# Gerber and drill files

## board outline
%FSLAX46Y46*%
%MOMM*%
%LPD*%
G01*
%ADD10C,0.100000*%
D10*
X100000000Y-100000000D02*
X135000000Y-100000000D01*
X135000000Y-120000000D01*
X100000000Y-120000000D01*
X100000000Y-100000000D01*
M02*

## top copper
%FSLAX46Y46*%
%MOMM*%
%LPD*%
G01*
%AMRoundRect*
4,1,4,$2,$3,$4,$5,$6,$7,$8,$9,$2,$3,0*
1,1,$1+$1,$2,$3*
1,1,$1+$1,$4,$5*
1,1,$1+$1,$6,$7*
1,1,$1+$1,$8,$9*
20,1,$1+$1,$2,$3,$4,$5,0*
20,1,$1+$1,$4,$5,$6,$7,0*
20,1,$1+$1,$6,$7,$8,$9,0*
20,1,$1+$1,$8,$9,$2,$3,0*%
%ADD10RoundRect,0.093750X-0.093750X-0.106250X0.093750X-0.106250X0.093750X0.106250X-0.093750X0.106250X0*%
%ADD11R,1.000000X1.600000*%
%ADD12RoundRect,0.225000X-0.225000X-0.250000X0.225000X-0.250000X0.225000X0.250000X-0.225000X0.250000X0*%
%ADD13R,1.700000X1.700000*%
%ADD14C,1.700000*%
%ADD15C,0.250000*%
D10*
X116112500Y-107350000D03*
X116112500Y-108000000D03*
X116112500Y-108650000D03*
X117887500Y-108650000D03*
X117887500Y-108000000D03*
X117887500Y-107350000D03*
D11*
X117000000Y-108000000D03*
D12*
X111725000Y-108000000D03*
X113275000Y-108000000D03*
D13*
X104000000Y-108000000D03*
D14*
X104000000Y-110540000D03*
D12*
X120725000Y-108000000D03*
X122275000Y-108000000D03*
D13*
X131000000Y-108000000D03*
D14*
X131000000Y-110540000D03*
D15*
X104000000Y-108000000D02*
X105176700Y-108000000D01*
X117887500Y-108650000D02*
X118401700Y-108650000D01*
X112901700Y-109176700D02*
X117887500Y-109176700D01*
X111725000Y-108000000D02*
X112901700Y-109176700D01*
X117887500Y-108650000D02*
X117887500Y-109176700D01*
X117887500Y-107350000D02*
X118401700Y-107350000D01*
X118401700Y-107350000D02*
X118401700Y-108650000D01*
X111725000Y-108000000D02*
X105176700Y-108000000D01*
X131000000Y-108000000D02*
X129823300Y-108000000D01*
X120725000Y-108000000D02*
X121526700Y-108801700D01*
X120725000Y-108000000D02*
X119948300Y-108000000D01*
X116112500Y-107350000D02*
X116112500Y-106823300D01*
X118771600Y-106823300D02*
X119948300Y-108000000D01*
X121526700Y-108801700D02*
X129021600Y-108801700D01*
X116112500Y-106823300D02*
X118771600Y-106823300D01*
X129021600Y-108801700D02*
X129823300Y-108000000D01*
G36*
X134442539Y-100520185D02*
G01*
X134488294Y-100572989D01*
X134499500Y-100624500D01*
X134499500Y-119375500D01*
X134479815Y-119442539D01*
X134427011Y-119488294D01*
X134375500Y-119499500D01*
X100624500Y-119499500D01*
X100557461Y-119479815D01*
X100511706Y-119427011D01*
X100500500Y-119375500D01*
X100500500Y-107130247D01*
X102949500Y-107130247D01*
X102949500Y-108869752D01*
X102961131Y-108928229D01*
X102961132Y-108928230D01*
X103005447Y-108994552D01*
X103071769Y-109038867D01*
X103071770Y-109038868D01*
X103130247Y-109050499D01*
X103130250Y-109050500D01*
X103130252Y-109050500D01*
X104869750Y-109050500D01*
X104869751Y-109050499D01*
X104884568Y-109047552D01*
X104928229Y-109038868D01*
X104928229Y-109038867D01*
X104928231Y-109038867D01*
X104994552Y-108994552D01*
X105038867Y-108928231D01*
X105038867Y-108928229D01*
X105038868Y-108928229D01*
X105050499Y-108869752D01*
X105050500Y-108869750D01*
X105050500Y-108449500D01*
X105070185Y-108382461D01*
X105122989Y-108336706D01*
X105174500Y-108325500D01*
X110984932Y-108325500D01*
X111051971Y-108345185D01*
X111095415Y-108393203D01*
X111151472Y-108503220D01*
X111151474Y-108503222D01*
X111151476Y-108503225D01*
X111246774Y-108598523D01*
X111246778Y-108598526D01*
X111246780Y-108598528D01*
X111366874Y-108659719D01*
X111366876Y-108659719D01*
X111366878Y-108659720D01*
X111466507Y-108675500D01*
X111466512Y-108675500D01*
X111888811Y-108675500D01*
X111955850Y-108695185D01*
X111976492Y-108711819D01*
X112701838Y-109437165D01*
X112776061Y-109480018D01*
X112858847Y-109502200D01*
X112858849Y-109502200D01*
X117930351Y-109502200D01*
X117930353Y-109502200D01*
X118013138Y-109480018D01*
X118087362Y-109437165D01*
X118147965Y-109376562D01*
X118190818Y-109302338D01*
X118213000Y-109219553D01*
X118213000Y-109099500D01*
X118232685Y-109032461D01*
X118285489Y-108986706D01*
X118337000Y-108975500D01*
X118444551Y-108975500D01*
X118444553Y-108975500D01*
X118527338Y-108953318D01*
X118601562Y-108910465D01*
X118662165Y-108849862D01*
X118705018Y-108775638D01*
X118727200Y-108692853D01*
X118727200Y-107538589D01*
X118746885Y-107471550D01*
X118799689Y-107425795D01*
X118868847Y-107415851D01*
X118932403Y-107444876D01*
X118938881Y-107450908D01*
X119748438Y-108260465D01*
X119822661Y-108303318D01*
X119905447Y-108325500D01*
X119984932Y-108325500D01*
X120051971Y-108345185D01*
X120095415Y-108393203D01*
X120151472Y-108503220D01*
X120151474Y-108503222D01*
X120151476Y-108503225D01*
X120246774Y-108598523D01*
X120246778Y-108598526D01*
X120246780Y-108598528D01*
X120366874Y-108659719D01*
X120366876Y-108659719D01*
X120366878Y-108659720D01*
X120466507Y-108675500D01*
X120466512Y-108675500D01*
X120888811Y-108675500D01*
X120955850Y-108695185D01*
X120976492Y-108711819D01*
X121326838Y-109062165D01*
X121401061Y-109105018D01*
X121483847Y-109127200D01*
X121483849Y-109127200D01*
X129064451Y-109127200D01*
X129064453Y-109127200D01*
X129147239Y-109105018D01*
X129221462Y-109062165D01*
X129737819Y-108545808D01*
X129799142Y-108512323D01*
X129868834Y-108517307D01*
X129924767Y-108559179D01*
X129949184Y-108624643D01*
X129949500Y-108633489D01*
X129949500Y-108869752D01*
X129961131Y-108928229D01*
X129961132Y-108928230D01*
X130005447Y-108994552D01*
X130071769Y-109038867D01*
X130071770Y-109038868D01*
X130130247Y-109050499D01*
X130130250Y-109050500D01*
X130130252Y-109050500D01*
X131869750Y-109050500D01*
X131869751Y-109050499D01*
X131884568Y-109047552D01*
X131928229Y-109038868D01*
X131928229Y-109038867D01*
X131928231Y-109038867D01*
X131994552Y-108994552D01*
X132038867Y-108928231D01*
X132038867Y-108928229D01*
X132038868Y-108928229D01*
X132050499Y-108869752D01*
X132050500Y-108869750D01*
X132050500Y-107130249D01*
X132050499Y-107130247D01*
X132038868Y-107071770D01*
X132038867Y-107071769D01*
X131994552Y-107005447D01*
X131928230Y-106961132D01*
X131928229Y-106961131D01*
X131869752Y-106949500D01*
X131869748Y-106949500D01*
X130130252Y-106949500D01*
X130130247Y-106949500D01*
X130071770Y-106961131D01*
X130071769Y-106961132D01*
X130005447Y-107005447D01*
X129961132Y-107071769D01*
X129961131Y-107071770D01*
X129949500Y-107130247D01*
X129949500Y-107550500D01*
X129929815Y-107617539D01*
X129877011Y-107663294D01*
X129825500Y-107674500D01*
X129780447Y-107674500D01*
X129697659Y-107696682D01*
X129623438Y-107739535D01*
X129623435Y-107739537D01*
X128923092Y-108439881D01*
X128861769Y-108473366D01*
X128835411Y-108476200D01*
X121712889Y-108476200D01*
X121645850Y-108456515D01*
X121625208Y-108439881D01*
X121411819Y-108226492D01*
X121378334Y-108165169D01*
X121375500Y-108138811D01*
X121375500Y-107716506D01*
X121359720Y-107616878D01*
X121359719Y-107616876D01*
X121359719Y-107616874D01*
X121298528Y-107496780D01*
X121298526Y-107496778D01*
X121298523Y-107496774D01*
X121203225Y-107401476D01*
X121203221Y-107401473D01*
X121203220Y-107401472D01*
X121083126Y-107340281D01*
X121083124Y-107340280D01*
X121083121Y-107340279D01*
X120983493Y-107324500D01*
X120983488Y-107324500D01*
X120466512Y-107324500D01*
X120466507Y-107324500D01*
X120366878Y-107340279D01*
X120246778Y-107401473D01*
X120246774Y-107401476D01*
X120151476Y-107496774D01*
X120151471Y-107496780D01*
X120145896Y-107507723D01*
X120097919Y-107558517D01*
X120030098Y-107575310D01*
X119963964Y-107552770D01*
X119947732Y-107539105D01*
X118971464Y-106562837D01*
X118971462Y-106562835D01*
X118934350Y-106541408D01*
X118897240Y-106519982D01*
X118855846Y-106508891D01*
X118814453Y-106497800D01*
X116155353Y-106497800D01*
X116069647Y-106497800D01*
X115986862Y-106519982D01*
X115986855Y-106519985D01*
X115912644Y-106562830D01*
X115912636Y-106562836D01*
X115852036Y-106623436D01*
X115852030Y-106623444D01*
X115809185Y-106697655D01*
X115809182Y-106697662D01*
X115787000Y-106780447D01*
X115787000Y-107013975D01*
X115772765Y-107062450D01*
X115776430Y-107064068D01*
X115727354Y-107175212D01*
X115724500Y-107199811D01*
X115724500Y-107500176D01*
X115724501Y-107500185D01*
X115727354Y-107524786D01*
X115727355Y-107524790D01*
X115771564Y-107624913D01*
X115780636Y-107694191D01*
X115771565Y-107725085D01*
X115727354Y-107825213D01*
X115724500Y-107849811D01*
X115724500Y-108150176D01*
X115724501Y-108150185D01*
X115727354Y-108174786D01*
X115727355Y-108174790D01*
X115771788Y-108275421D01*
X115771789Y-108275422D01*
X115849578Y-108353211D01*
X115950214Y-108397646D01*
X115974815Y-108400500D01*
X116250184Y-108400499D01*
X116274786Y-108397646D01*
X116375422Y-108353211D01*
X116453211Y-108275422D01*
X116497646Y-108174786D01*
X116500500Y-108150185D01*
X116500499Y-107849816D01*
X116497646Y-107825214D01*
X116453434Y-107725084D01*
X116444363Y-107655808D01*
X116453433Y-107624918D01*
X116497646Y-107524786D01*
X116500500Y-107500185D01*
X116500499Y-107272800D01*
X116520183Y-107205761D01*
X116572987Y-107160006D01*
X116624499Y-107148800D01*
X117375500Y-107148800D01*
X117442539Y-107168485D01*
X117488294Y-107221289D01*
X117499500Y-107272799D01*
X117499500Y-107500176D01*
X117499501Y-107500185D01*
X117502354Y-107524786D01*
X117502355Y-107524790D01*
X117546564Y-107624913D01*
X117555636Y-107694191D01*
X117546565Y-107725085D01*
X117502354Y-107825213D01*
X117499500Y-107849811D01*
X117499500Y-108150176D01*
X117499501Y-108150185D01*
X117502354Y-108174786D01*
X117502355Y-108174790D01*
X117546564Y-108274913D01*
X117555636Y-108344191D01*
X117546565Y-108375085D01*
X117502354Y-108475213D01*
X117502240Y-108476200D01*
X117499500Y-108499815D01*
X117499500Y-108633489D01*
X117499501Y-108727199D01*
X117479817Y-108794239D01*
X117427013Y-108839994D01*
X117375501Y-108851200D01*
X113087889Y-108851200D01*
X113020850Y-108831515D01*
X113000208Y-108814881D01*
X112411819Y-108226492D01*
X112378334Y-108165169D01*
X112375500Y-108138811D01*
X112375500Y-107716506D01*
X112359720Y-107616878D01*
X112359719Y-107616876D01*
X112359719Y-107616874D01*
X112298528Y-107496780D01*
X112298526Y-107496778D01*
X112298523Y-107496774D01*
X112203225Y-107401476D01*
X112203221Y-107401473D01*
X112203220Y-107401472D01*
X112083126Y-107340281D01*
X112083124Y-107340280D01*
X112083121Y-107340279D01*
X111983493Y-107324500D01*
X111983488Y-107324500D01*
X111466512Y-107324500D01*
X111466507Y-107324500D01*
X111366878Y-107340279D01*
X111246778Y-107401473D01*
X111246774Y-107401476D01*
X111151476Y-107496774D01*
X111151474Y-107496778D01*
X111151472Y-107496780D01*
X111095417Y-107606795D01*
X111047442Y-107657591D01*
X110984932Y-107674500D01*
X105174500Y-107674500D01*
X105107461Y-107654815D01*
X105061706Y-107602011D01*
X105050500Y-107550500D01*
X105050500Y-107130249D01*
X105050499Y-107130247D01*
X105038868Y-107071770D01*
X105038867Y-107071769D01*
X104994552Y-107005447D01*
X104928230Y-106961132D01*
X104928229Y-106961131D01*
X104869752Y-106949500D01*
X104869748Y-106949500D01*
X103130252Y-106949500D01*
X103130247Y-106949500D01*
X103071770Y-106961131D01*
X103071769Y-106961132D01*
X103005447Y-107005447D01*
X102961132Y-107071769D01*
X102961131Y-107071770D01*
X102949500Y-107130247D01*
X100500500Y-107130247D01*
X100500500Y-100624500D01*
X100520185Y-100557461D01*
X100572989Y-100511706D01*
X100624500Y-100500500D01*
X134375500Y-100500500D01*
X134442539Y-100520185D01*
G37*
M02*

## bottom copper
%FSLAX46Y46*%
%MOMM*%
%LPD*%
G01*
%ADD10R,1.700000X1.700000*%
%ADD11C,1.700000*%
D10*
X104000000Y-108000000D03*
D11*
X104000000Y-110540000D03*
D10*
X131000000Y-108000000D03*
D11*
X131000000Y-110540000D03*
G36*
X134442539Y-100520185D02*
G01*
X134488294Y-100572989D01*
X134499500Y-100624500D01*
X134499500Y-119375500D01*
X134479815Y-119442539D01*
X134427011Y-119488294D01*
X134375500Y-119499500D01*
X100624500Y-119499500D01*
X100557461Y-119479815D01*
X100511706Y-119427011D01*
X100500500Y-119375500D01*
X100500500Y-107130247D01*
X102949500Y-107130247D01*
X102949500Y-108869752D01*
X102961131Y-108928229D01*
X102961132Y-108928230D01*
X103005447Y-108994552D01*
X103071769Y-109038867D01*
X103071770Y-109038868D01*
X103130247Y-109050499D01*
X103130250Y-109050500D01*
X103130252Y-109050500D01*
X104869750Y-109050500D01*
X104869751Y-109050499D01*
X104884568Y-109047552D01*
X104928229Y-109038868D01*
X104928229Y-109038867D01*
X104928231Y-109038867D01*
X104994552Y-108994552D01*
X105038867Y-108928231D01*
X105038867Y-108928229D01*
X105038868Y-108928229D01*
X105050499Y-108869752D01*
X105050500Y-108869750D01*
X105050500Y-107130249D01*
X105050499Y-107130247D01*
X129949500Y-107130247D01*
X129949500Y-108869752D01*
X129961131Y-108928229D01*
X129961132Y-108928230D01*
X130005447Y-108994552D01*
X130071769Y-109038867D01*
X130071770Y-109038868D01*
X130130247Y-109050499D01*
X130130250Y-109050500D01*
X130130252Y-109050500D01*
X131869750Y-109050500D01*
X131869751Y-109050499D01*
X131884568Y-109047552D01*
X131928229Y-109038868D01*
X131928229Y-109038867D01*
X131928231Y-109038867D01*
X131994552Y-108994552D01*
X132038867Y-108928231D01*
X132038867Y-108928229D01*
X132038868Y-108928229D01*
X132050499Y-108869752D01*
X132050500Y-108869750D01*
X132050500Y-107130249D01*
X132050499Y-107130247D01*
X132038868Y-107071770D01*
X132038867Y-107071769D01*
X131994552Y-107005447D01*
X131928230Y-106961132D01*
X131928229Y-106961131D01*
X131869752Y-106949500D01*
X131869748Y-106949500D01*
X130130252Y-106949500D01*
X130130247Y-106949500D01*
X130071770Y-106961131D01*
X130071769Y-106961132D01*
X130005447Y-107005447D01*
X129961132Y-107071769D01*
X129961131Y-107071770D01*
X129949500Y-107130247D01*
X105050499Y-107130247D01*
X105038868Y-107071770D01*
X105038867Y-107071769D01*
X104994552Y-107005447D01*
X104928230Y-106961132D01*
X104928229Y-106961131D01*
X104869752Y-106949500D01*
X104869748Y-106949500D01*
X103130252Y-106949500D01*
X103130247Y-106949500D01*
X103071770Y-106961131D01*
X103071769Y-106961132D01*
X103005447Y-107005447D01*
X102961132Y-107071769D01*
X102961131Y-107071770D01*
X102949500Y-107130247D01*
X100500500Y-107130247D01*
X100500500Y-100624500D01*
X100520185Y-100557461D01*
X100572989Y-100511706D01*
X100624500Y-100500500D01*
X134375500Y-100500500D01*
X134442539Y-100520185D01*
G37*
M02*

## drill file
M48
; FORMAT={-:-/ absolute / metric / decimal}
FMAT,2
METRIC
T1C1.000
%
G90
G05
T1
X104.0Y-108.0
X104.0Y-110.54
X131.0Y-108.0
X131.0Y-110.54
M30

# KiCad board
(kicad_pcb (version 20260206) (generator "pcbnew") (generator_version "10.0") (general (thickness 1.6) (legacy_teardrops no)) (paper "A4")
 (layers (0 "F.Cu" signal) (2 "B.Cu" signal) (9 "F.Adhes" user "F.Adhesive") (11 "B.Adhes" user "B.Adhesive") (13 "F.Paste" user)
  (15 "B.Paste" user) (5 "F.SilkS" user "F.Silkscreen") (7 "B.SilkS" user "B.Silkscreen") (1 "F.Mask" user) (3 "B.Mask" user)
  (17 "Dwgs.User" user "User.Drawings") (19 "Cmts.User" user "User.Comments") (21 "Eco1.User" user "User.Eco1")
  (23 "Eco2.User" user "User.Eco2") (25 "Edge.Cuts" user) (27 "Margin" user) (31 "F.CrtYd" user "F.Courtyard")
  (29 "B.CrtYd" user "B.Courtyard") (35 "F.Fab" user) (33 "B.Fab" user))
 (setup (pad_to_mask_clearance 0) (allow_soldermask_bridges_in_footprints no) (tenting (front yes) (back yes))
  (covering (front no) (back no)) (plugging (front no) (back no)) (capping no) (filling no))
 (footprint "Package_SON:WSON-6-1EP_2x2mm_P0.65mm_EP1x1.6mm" (layer "F.Cu") (at 117 108)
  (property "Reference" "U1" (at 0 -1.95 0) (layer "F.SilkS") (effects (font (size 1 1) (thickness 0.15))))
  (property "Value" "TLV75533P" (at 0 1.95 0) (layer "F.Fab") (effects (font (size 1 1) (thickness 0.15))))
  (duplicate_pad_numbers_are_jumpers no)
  (pad "" smd roundrect (at 0 -0.4) (size 0.81 0.64) (layers "F.Paste") (roundrect_rratio 0.25))
  (pad "" smd roundrect (at 0 0.4) (size 0.81 0.64) (layers "F.Paste") (roundrect_rratio 0.25))
  (pad "1" smd roundrect (at -0.8875 -0.65) (size 0.375 0.4) (layers "F.Cu" "F.Mask" "F.Paste") (roundrect_rratio 0.25) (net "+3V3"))
  (pad "2" smd roundrect (at -0.8875 0) (size 0.375 0.4) (layers "F.Cu" "F.Mask" "F.Paste") (roundrect_rratio 0.25)
   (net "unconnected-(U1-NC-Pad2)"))
  (pad "3" smd roundrect (at -0.8875 0.65) (size 0.375 0.4) (layers "F.Cu" "F.Mask" "F.Paste") (roundrect_rratio 0.25) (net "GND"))
  (pad "4" smd roundrect (at 0.8875 0.65) (size 0.375 0.4) (layers "F.Cu" "F.Mask" "F.Paste") (roundrect_rratio 0.25) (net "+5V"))
  (pad "5" smd roundrect (at 0.8875 0) (size 0.375 0.4) (layers "F.Cu" "F.Mask" "F.Paste") (roundrect_rratio 0.25)
   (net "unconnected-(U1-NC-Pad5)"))
  (pad "6" smd roundrect (at 0.8875 -0.65) (size 0.375 0.4) (layers "F.Cu" "F.Mask" "F.Paste") (roundrect_rratio 0.25) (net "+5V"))
  (pad "7" smd rect (at 0 0) (size 1 1.6) (layers "F.Cu" "F.Mask") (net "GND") (zone_connect 2)))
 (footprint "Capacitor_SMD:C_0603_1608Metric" (layer "F.Cu") (at 112.5 108)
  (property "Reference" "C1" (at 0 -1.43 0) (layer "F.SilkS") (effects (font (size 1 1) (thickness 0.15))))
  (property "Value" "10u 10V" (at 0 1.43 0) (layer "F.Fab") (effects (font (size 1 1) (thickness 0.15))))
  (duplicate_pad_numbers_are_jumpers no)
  (pad "1" smd roundrect (at -0.775 0) (size 0.9 0.95) (layers "F.Cu" "F.Mask" "F.Paste") (roundrect_rratio 0.25) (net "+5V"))
  (pad "2" smd roundrect (at 0.775 0) (size 0.9 0.95) (layers "F.Cu" "F.Mask" "F.Paste") (roundrect_rratio 0.25) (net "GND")))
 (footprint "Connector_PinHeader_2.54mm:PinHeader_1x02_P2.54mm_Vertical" (layer "F.Cu") (at 104 108)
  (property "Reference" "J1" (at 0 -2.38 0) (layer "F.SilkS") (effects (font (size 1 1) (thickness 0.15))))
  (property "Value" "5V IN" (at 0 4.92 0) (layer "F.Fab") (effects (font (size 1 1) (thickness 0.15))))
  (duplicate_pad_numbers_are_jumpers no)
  (pad "1" thru_hole rect (at 0 0) (size 1.7 1.7) (drill 1) (layers "*.Cu" "*.Mask") (remove_unused_layers no) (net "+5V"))
  (pad "2" thru_hole circle (at 0 2.54) (size 1.7 1.7) (drill 1) (layers "*.Cu" "*.Mask") (remove_unused_layers no) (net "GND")))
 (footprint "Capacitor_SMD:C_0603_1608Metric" (layer "F.Cu") (at 121.5 108)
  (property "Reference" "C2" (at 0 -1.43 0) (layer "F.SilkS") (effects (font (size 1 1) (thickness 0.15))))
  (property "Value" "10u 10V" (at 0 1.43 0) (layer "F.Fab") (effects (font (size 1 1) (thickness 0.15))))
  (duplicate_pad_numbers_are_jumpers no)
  (pad "1" smd roundrect (at -0.775 0) (size 0.9 0.95) (layers "F.Cu" "F.Mask" "F.Paste") (roundrect_rratio 0.25) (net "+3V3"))
  (pad "2" smd roundrect (at 0.775 0) (size 0.9 0.95) (layers "F.Cu" "F.Mask" "F.Paste") (roundrect_rratio 0.25) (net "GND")))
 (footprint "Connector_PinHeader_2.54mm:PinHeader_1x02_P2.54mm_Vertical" (layer "F.Cu") (at 131 108)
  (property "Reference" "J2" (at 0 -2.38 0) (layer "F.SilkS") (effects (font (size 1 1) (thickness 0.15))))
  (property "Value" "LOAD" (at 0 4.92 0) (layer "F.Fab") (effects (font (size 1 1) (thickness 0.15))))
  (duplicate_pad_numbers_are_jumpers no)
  (pad "1" thru_hole rect (at 0 0) (size 1.7 1.7) (drill 1) (layers "*.Cu" "*.Mask") (remove_unused_layers no) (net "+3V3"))
  (pad "2" thru_hole circle (at 0 2.54) (size 1.7 1.7) (drill 1) (layers "*.Cu" "*.Mask") (remove_unused_layers no) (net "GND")))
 (gr_rect (start 100 100) (end 135 120) (stroke (width 0.1) (type default)) (fill no) (layer "Edge.Cuts"))
 (segment (start 104 108) (end 105.1767 108) (width 0.25) (layer "F.Cu") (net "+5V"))
 (segment (start 117.8875 108.65) (end 118.4017 108.65) (width 0.25) (layer "F.Cu") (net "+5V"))
 (segment (start 112.9017 109.1767) (end 117.8875 109.1767) (width 0.25) (layer "F.Cu") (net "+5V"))
 (segment (start 111.725 108) (end 112.9017 109.1767) (width 0.25) (layer "F.Cu") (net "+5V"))
 (segment (start 117.8875 108.65) (end 117.8875 109.1767) (width 0.25) (layer "F.Cu") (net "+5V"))
 (segment (start 117.8875 107.35) (end 118.4017 107.35) (width 0.25) (layer "F.Cu") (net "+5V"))
 (segment (start 118.4017 107.35) (end 118.4017 108.65) (width 0.25) (layer "F.Cu") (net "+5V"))
 (segment (start 111.725 108) (end 105.1767 108) (width 0.25) (layer "F.Cu") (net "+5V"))
 (segment (start 131 108) (end 129.8233 108) (width 0.25) (layer "F.Cu") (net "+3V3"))
 (segment (start 120.725 108) (end 121.5267 108.8017) (width 0.25) (layer "F.Cu") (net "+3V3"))
 (segment (start 120.725 108) (end 119.9483 108) (width 0.25) (layer "F.Cu") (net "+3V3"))
 (segment (start 116.1125 107.35) (end 116.1125 106.8233) (width 0.25) (layer "F.Cu") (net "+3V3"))
 (segment (start 118.7716 106.8233) (end 119.9483 108) (width 0.25) (layer "F.Cu") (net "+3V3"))
 (segment (start 121.5267 108.8017) (end 129.0216 108.8017) (width 0.25) (layer "F.Cu") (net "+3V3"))
 (segment (start 116.1125 106.8233) (end 118.7716 106.8233) (width 0.25) (layer "F.Cu") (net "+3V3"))
 (segment (start 129.0216 108.8017) (end 129.8233 108) (width 0.25) (layer "F.Cu") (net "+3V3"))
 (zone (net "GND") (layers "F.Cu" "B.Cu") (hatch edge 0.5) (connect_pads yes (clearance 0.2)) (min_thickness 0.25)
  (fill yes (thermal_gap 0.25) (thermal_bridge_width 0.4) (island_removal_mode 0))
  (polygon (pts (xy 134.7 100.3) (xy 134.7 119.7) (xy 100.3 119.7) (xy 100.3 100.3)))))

